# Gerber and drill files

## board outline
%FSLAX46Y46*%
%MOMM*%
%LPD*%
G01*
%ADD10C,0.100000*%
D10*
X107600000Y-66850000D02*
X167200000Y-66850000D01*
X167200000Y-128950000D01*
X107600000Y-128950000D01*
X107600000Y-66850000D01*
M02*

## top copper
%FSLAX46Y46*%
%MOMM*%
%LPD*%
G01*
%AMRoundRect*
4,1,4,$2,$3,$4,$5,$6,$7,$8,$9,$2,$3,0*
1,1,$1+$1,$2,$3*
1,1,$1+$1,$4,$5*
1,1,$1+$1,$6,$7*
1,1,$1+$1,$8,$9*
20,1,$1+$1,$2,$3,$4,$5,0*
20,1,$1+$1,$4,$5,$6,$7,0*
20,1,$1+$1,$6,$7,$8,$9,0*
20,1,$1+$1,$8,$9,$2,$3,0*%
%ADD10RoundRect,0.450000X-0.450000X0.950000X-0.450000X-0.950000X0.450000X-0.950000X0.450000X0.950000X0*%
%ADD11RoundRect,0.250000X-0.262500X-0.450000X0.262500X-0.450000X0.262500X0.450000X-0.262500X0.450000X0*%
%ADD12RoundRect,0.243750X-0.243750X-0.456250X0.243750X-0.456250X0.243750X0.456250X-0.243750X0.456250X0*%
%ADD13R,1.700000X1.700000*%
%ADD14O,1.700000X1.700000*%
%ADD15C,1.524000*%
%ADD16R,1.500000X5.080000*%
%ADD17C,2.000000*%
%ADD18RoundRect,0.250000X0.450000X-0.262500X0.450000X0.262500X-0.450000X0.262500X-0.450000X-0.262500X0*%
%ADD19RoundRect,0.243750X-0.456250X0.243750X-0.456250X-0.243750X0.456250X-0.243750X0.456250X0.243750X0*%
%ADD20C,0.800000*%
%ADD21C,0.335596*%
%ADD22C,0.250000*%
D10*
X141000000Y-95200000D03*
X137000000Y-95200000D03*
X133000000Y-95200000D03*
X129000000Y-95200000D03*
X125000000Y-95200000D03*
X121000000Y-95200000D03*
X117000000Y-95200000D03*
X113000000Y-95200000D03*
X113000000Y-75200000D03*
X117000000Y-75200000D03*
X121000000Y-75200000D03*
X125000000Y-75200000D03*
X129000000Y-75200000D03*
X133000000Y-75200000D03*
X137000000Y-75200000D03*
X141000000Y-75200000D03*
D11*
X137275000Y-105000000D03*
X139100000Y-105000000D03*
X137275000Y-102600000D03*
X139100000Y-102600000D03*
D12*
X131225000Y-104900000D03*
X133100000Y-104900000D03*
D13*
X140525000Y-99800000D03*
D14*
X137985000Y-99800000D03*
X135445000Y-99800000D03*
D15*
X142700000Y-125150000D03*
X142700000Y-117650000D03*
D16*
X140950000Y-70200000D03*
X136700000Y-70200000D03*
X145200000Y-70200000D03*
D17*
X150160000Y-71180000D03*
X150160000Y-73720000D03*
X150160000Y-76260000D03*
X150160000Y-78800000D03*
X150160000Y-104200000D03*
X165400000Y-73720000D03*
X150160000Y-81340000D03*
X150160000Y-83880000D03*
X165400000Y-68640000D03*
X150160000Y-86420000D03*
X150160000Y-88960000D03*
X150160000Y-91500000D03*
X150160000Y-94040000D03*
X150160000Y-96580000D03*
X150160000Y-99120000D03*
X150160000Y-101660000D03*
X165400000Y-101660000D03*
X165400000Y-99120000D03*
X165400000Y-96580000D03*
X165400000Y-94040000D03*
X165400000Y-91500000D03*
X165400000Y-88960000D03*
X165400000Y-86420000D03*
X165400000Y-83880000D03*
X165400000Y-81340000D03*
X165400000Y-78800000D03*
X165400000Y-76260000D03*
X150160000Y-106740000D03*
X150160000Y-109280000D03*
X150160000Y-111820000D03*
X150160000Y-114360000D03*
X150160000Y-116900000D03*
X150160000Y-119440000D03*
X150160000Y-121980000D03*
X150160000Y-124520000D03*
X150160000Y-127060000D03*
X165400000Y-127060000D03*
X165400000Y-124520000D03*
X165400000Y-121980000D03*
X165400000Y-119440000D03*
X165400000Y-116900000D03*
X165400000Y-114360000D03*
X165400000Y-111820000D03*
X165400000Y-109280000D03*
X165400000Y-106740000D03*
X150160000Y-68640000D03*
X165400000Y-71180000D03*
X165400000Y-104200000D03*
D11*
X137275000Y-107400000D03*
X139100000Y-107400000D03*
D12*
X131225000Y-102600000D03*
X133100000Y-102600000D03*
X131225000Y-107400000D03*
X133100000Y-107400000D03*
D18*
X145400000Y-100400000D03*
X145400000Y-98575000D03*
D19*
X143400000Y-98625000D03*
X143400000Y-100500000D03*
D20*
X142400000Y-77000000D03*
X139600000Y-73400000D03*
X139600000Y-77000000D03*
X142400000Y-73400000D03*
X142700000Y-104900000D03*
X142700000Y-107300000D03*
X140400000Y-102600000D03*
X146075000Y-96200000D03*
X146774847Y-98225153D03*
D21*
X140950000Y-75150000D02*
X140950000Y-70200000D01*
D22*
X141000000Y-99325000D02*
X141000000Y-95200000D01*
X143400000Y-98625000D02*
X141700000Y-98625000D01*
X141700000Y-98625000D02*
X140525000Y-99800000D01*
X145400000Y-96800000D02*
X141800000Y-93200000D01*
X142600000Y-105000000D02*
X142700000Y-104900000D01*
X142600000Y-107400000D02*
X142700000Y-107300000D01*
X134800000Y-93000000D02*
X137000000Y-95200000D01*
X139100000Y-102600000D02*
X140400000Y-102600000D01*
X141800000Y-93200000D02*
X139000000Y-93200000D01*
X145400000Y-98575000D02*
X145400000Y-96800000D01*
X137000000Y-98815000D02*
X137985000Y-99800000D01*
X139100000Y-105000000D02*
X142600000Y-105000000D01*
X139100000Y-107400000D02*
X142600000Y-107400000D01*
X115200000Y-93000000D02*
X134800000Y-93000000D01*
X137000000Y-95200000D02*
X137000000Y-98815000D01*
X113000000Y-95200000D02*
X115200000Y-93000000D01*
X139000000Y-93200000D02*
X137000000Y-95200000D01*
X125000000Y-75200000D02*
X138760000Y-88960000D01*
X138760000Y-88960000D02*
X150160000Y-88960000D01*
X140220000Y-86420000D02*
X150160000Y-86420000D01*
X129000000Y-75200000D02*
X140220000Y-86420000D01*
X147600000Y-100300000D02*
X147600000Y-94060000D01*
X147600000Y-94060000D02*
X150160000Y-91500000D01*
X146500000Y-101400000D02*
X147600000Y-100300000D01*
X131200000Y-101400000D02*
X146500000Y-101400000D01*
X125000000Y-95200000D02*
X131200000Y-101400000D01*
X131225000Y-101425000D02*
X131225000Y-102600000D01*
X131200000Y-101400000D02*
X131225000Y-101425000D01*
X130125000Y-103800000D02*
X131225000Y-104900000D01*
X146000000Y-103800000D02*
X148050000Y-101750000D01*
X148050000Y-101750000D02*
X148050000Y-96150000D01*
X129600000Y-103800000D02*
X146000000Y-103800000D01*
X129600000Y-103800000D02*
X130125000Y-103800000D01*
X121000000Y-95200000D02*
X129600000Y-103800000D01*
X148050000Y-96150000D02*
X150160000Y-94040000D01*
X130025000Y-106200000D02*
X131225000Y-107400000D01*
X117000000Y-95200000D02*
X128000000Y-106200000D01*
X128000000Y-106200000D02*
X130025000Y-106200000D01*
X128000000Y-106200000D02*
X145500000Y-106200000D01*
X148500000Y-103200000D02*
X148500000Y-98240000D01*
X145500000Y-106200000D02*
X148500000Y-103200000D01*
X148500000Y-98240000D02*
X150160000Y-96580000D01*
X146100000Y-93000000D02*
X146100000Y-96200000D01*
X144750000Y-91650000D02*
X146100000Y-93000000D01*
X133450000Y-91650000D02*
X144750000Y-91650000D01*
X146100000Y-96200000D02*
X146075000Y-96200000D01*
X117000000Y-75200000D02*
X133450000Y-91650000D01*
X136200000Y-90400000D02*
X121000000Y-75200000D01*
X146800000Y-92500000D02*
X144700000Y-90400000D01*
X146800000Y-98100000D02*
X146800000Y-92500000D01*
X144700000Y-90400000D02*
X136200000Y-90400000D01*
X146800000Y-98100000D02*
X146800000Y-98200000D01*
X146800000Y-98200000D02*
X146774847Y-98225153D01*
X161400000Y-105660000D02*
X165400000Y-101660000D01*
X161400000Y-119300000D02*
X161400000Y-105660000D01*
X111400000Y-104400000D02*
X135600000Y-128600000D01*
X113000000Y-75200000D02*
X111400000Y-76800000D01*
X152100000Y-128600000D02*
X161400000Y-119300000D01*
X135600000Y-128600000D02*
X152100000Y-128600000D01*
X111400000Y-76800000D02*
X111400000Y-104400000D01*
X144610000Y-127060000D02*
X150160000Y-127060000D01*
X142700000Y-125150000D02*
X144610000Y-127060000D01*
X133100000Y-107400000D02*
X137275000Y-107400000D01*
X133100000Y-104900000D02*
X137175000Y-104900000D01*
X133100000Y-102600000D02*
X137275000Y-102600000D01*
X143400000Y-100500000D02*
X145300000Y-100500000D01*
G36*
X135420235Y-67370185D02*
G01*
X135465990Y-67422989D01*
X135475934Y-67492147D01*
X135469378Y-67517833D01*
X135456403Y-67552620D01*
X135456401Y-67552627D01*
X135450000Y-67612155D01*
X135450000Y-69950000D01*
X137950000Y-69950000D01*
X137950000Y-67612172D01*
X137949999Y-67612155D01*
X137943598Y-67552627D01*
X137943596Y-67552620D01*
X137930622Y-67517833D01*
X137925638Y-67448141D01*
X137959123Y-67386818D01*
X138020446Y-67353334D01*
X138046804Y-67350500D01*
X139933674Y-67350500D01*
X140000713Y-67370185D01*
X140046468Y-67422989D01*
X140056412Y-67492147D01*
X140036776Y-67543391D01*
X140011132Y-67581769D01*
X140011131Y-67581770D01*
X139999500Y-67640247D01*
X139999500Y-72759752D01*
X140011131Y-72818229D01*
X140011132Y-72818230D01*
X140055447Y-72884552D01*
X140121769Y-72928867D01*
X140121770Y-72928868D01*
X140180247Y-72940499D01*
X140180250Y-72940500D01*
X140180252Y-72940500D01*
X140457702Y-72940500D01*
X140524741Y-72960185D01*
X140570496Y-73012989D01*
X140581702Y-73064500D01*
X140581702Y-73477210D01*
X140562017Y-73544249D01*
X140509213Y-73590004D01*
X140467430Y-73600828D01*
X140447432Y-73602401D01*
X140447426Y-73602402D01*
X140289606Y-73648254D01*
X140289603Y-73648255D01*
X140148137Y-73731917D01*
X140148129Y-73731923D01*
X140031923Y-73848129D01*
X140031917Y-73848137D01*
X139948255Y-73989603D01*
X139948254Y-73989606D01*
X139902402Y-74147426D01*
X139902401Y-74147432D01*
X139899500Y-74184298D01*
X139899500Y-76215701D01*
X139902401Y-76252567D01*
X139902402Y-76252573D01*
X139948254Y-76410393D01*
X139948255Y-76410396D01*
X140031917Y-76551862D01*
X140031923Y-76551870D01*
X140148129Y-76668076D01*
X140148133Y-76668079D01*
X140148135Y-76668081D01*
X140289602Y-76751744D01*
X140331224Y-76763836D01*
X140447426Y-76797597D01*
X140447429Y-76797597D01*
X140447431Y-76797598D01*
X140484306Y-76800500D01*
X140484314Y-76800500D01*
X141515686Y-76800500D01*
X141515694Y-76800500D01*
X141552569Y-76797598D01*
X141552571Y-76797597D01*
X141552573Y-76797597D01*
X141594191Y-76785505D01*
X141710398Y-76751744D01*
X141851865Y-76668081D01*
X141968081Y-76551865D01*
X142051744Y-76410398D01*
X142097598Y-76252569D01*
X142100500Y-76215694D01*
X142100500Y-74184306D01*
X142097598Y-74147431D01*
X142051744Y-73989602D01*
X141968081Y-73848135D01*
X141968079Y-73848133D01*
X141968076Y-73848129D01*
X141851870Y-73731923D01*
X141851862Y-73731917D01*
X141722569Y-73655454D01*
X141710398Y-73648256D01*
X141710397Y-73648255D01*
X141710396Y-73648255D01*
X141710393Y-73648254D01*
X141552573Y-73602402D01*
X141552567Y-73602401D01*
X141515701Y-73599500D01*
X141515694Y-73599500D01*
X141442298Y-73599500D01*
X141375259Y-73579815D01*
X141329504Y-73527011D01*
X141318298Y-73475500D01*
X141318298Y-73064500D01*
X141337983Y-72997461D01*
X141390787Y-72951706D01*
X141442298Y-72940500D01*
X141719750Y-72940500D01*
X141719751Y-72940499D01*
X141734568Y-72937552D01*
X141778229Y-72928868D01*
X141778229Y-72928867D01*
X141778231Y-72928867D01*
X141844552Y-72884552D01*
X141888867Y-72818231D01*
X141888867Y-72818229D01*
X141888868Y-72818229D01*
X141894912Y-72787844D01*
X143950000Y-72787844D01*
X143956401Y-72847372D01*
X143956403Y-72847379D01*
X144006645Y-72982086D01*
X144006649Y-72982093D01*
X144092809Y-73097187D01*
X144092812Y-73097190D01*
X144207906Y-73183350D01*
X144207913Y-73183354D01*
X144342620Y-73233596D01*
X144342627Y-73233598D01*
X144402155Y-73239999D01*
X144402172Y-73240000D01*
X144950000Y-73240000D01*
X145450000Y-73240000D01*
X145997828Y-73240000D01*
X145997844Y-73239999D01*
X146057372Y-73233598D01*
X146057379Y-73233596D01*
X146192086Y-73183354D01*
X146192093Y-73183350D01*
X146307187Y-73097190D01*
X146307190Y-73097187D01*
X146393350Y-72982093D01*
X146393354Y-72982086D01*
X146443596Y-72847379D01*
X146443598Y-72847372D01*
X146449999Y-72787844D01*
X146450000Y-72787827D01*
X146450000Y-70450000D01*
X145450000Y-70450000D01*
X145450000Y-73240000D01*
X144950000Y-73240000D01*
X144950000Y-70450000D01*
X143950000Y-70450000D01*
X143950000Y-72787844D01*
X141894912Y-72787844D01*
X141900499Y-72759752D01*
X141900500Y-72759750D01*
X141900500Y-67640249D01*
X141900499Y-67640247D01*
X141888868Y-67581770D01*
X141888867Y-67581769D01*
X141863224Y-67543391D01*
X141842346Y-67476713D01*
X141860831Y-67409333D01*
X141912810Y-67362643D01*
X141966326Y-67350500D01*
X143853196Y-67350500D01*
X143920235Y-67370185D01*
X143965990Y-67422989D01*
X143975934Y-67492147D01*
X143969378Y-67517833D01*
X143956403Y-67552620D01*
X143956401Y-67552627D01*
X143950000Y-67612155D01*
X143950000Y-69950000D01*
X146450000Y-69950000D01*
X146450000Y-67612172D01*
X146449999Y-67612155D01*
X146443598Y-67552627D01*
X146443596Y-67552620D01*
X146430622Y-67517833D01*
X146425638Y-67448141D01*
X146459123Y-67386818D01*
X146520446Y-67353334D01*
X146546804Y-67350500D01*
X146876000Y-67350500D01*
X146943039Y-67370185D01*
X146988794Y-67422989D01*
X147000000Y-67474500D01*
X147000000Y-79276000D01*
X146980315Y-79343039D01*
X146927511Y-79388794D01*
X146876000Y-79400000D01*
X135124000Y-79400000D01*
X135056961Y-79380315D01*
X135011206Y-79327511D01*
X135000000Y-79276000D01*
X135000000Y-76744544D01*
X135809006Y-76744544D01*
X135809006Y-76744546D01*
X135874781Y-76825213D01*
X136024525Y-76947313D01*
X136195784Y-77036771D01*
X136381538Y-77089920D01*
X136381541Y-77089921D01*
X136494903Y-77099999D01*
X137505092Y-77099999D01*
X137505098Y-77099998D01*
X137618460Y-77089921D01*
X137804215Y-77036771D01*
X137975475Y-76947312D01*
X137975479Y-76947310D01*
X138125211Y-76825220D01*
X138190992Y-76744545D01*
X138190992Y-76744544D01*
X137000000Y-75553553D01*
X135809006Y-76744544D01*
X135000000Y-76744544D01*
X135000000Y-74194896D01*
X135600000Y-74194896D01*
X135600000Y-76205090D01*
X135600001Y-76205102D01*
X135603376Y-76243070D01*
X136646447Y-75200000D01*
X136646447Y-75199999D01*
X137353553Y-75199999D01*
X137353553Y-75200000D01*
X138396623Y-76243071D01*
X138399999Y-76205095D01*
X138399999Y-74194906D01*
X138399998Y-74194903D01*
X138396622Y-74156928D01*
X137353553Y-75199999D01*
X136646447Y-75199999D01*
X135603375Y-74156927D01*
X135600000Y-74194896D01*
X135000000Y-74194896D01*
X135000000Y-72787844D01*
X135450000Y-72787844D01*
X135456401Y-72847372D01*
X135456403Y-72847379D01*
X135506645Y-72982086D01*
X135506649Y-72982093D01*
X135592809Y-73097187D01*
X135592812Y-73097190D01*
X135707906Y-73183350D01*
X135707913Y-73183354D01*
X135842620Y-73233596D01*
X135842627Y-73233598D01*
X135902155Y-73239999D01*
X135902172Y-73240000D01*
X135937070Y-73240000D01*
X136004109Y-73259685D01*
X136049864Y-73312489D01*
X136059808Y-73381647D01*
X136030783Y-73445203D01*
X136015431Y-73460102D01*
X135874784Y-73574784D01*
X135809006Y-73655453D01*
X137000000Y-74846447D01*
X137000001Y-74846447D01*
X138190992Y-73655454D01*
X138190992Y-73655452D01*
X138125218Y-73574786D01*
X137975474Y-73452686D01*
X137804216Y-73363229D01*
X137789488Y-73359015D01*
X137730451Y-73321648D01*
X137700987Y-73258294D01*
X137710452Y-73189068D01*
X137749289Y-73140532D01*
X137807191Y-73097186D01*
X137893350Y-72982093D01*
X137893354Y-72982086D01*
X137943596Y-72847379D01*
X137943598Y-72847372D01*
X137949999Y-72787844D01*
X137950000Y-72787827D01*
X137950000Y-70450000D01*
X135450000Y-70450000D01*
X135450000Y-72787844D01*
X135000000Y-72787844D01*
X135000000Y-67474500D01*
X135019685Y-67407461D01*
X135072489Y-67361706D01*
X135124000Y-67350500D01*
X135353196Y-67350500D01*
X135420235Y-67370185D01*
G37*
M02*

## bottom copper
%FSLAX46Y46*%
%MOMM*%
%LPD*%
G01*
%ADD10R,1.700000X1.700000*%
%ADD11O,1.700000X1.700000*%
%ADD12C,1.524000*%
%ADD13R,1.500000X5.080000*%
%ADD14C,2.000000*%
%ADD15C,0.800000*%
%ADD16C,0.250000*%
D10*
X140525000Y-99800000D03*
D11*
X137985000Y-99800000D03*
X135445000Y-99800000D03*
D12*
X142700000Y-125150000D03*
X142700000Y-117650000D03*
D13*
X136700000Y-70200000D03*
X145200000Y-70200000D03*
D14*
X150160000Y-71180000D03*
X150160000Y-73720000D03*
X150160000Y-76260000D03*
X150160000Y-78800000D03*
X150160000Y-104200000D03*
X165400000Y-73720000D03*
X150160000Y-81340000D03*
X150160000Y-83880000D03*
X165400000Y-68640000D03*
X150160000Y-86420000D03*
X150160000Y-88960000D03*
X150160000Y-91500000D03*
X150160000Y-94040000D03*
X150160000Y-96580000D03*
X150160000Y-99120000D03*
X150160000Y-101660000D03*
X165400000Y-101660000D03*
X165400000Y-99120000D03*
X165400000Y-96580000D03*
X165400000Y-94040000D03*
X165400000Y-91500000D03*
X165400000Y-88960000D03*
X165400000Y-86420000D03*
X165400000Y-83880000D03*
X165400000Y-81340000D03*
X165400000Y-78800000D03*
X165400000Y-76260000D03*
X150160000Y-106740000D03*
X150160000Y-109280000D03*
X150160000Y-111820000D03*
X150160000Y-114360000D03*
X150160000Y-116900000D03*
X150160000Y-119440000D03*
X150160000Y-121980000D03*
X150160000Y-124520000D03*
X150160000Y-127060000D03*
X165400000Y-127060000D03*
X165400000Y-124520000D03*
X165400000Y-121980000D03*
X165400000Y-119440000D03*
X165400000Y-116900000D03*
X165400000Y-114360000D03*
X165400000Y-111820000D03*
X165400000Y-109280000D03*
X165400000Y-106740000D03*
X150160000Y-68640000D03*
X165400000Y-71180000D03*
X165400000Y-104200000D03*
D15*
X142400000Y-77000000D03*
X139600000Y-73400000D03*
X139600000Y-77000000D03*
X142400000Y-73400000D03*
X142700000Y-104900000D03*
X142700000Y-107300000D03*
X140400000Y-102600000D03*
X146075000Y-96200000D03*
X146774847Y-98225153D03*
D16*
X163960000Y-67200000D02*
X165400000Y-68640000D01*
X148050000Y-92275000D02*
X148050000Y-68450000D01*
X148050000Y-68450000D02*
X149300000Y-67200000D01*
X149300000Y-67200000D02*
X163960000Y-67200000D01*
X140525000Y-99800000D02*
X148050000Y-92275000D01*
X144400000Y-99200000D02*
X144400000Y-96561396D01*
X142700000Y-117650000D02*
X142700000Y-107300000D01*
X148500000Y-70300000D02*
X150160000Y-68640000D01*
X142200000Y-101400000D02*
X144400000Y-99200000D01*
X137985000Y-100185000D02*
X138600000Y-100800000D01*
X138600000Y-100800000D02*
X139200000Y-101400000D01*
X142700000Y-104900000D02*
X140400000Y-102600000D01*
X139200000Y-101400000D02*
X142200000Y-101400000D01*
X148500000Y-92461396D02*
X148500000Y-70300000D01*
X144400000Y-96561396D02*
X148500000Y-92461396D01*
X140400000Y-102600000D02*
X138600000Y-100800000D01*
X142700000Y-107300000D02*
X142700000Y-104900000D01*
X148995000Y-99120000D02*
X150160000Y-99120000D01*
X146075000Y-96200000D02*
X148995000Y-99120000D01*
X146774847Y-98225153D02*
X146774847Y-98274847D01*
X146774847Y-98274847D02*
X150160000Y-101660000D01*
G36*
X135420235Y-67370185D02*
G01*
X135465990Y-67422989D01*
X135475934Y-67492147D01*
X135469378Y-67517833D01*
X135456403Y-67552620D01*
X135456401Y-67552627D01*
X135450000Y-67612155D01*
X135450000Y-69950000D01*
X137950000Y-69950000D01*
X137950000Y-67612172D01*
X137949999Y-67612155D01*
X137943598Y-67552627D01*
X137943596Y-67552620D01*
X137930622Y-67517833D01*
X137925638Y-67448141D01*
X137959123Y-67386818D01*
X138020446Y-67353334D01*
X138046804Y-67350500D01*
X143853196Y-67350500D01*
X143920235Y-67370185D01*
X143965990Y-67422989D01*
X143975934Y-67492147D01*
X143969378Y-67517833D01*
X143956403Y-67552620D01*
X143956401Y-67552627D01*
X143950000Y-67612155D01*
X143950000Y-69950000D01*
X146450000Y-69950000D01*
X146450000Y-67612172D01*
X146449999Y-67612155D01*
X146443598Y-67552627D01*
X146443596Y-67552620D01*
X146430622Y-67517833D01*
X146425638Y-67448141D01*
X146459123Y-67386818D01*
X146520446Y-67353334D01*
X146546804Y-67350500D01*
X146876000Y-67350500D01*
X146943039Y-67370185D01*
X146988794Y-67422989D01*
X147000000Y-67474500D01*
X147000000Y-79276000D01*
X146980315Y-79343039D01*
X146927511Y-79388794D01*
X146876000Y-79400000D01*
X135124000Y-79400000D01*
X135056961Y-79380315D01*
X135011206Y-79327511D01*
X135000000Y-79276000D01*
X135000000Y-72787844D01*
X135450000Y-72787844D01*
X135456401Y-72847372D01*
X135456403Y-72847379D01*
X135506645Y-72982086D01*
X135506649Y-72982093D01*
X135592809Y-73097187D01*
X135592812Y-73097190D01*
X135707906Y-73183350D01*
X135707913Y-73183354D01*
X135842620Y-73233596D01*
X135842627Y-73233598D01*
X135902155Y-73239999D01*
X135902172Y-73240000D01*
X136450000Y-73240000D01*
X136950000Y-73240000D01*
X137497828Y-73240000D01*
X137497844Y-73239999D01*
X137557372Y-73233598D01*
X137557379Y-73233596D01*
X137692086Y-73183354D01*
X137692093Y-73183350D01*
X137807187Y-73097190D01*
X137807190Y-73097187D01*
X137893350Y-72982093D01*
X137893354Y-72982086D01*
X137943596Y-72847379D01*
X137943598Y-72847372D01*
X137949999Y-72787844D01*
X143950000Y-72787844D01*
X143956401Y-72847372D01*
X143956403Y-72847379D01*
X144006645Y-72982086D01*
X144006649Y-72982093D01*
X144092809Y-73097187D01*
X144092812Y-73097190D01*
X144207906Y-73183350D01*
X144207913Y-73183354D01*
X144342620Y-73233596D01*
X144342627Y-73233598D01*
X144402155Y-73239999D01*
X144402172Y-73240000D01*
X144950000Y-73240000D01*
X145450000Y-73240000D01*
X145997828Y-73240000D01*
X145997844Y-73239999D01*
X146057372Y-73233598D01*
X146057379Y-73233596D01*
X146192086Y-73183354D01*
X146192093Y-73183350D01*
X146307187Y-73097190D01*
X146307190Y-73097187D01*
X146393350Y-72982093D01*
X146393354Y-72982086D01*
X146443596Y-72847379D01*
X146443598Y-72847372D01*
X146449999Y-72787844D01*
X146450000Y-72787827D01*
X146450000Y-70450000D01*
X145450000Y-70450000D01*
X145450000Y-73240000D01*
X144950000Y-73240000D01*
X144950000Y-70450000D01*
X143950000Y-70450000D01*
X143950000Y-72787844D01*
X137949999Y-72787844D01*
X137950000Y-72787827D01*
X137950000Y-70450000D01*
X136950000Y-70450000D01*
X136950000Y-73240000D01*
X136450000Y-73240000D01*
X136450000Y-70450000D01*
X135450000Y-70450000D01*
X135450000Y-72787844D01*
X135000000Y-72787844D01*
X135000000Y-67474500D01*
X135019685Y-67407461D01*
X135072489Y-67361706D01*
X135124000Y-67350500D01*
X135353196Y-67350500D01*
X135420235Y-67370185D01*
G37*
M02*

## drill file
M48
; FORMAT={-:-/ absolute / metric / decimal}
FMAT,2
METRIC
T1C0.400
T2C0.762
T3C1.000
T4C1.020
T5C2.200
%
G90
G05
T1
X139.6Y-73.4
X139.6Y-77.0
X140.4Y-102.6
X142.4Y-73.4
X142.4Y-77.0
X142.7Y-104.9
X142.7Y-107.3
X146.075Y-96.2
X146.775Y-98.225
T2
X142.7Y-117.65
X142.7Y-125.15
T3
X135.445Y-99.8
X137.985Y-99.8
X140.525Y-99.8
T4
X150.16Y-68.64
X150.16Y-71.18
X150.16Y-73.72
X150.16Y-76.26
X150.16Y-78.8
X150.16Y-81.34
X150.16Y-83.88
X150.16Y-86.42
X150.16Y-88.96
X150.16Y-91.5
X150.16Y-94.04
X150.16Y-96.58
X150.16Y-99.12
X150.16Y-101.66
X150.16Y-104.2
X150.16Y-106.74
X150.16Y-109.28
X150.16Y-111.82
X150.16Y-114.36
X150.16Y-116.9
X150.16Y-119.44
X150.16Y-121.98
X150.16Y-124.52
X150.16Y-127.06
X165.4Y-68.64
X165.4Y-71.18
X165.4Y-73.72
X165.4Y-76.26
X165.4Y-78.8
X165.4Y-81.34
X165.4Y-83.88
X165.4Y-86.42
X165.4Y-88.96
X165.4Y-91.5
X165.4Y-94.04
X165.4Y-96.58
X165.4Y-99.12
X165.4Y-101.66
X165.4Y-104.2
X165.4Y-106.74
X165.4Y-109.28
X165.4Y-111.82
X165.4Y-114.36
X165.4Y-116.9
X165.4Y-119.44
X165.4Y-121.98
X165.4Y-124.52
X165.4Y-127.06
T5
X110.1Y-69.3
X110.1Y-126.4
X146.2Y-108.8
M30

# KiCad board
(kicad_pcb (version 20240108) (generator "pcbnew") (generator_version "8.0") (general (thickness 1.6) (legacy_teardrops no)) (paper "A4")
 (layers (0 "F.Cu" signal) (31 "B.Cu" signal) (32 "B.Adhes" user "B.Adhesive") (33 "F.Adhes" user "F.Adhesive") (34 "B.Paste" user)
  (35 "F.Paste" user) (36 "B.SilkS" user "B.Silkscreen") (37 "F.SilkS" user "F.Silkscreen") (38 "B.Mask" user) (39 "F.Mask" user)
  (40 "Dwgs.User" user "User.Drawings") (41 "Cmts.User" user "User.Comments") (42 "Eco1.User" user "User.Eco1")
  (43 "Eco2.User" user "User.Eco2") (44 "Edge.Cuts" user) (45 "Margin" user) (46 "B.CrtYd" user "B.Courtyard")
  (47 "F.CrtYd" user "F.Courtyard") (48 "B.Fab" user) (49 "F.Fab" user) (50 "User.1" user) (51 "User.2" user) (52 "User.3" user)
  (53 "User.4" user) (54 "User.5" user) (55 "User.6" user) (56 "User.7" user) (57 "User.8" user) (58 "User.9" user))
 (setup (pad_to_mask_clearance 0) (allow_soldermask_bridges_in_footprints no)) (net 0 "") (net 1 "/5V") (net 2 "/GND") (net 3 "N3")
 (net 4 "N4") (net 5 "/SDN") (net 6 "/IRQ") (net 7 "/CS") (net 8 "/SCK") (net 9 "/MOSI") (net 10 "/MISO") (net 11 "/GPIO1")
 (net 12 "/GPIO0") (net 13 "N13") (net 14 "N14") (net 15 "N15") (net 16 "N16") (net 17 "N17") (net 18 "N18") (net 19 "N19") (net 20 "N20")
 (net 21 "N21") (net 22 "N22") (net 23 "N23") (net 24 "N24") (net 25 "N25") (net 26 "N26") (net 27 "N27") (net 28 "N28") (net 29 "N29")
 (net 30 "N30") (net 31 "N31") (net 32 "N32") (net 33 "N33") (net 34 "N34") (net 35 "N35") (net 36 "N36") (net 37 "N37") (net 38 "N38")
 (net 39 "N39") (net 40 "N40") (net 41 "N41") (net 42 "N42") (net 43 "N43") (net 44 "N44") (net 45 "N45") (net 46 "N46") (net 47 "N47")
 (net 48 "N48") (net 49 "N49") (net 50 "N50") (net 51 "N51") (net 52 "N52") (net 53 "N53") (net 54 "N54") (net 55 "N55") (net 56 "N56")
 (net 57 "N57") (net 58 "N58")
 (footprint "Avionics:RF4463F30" (layer "F.Cu") (at 127 85.2 180)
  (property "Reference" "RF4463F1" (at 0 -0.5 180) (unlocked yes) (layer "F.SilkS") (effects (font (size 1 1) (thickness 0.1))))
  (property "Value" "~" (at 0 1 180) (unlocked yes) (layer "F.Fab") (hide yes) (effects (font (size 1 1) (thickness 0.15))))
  (pad "1" smd roundrect (at -14 -10 270) (size 2.8 1.8) (layers "F.Cu" "F.Paste" "F.Mask") (roundrect_rratio 0.25) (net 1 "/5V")
   (thermal_bridge_angle 45))
  (pad "2" smd roundrect (at -10 -10 270) (size 2.8 1.8) (layers "F.Cu" "F.Paste" "F.Mask") (roundrect_rratio 0.25) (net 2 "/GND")
   (thermal_bridge_angle 45))
  (pad "3" smd roundrect (at -6 -10 270) (size 2.8 1.8) (layers "F.Cu" "F.Paste" "F.Mask") (roundrect_rratio 0.25) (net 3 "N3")
   (thermal_bridge_angle 45))
  (pad "4" smd roundrect (at -2 -10 270) (size 2.8 1.8) (layers "F.Cu" "F.Paste" "F.Mask") (roundrect_rratio 0.25) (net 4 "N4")
   (thermal_bridge_angle 45))
  (pad "5" smd roundrect (at 2 -10 270) (size 2.8 1.8) (layers "F.Cu" "F.Paste" "F.Mask") (roundrect_rratio 0.25) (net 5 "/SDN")
   (thermal_bridge_angle 45))
  (pad "6" smd roundrect (at 6 -10 270) (size 2.8 1.8) (layers "F.Cu" "F.Paste" "F.Mask") (roundrect_rratio 0.25) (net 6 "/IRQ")
   (thermal_bridge_angle 45))
  (pad "7" smd roundrect (at 10 -10 270) (size 2.8 1.8) (layers "F.Cu" "F.Paste" "F.Mask") (roundrect_rratio 0.25) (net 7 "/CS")
   (thermal_bridge_angle 45))
  (pad "8" smd roundrect (at 14 -10 270) (size 2.8 1.8) (layers "F.Cu" "F.Paste" "F.Mask") (roundrect_rratio 0.25) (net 2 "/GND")
   (thermal_bridge_angle 45))
  (pad "9" smd roundrect (at 14 10 270) (size 2.8 1.8) (layers "F.Cu" "F.Paste" "F.Mask") (roundrect_rratio 0.25) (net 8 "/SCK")
   (thermal_bridge_angle 45))
  (pad "10" smd roundrect (at 10 10 270) (size 2.8 1.8) (layers "F.Cu" "F.Paste" "F.Mask") (roundrect_rratio 0.25) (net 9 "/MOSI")
   (thermal_bridge_angle 45))
  (pad "11" smd roundrect (at 6 10 270) (size 2.8 1.8) (layers "F.Cu" "F.Paste" "F.Mask") (roundrect_rratio 0.25) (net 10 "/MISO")
   (thermal_bridge_angle 45))
  (pad "12" smd roundrect (at 2 10 270) (size 2.8 1.8) (layers "F.Cu" "F.Paste" "F.Mask") (roundrect_rratio 0.25) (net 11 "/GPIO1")
   (thermal_bridge_angle 45))
  (pad "13" smd roundrect (at -2 10 270) (size 2.8 1.8) (layers "F.Cu" "F.Paste" "F.Mask") (roundrect_rratio 0.25) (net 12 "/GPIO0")
   (thermal_bridge_angle 45))
  (pad "14" smd roundrect (at -6 10 270) (size 2.8 1.8) (layers "F.Cu" "F.Paste" "F.Mask") (roundrect_rratio 0.25) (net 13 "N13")
   (thermal_bridge_angle 45))
  (pad "15" smd roundrect (at -10 10 270) (size 2.8 1.8) (layers "F.Cu" "F.Paste" "F.Mask") (roundrect_rratio 0.25) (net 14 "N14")
   (thermal_bridge_angle 45))
  (pad "16" smd roundrect (at -14 10 270) (size 2.8 1.8) (layers "F.Cu" "F.Paste" "F.Mask") (roundrect_rratio 0.25) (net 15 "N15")
   (thermal_bridge_angle 45)))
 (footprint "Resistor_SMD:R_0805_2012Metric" (layer "F.Cu") (at 138.1875 105)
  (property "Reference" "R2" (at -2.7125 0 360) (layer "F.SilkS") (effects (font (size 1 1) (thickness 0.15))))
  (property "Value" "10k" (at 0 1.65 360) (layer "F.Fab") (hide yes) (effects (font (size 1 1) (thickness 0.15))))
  (pad "1" smd roundrect (at -0.9125 0) (size 1.025 1.4) (layers "F.Cu" "F.Paste" "F.Mask") (roundrect_rratio 0.243902) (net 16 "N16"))
  (pad "2" smd roundrect (at 0.9125 0) (size 1.025 1.4) (layers "F.Cu" "F.Paste" "F.Mask") (roundrect_rratio 0.243902) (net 2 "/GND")))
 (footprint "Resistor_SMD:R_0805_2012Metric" (layer "F.Cu") (at 138.1875 102.6)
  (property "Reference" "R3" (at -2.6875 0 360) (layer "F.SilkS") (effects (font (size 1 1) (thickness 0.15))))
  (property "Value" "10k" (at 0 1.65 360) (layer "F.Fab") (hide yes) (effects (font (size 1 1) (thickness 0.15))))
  (pad "1" smd roundrect (at -0.9125 0) (size 1.025 1.4) (layers "F.Cu" "F.Paste" "F.Mask") (roundrect_rratio 0.243902) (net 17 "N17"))
  (pad "2" smd roundrect (at 0.9125 0) (size 1.025 1.4) (layers "F.Cu" "F.Paste" "F.Mask") (roundrect_rratio 0.243902) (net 2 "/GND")))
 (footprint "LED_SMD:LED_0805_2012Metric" (layer "F.Cu") (at 132.1625 104.9)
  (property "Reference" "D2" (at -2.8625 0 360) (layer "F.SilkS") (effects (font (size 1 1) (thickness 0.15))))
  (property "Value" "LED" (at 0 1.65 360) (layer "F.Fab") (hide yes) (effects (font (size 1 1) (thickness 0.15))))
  (pad "1" smd roundrect (at -0.9375 0) (size 0.975 1.4) (layers "F.Cu" "F.Paste" "F.Mask") (roundrect_rratio 0.25) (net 6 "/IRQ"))
  (pad "2" smd roundrect (at 0.9375 0) (size 0.975 1.4) (layers "F.Cu" "F.Paste" "F.Mask") (roundrect_rratio 0.25) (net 16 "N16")))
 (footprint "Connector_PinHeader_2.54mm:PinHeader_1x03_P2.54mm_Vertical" (layer "F.Cu") (at 140.525 99.8 -90)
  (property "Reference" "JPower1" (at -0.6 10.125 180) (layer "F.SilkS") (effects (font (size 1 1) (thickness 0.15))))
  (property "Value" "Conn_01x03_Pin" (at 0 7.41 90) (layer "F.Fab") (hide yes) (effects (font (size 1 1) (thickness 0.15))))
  (pad "1" thru_hole rect (at 0 0 270) (size 1.7 1.7) (drill 1) (layers "*.Cu" "*.Mask") (remove_unused_layers no) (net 1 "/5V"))
  (pad "2" thru_hole oval (at 0 2.54 270) (size 1.7 1.7) (drill 1) (layers "*.Cu" "*.Mask") (remove_unused_layers no) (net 2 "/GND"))
  (pad "3" thru_hole oval (at 0 5.08 270) (size 1.7 1.7) (drill 1) (layers "*.Cu" "*.Mask") (remove_unused_layers no) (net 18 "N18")))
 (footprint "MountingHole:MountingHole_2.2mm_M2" (layer "F.Cu") (at 110.1 69.3)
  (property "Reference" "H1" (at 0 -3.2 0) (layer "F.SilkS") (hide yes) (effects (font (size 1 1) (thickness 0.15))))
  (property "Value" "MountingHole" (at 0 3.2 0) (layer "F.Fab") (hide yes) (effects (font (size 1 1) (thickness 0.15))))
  (pad "" np_thru_hole circle (at 0 0) (size 2.2 2.2) (drill 2.2) (layers "*.Cu" "*.Mask")))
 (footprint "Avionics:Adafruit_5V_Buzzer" (layer "F.Cu") (at 147.2 121.4 90)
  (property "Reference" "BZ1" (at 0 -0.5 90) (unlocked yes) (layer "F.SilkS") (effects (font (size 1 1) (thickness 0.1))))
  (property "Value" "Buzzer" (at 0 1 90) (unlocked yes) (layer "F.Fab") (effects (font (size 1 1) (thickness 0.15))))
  (pad "1" thru_hole circle (at -3.75 -4.5 90) (size 1.524 1.524) (drill 0.762) (layers "*.Cu" "*.Mask") (remove_unused_layers no)
   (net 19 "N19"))
  (pad "2" thru_hole circle (at 3.75 -4.5 90) (size 1.524 1.524) (drill 0.762) (layers "*.Cu" "*.Mask") (remove_unused_layers no)
   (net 2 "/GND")))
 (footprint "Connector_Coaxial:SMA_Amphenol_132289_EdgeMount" (layer "F.Cu") (at 140.95 70.2 90)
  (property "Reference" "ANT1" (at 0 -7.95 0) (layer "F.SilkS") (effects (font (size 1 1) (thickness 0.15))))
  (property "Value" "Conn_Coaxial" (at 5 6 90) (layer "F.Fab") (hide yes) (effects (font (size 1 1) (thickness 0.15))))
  (pad "1" smd rect (at 0 0 180) (size 1.5 5.08) (layers "F.Cu" "F.Paste" "F.Mask") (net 15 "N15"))
  (pad "2" smd rect (at 0 -4.25 180) (size 1.5 5.08) (layers "F.Cu" "F.Paste" "F.Mask") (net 14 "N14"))
  (pad "2" smd rect (at 0 -4.25 180) (size 1.5 5.08) (layers "B.Cu" "B.Paste" "B.Mask") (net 14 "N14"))
  (pad "2" smd rect (at 0 4.25 180) (size 1.5 5.08) (layers "F.Cu" "F.Paste" "F.Mask") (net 14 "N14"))
  (pad "2" smd rect (at 0 4.25 180) (size 1.5 5.08) (layers "B.Cu" "B.Paste" "B.Mask") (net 14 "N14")))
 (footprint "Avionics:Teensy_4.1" (layer "F.Cu") (at 157.78 97.85)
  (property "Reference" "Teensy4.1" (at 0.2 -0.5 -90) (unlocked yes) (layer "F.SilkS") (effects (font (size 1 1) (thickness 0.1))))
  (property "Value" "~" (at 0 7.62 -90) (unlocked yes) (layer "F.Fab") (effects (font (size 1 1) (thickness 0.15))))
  (pad "0" thru_hole circle (at -7.62 -26.67) (size 2 2) (drill 1.02) (layers "*.Cu" "*.Mask") (remove_unused_layers no) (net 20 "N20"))
  (pad "1" thru_hole circle (at -7.62 -24.13) (size 2 2) (drill 1.02) (layers "*.Cu" "*.Mask") (remove_unused_layers no) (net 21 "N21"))
  (pad "2" thru_hole circle (at -7.62 -21.59) (size 2 2) (drill 1.02) (layers "*.Cu" "*.Mask") (remove_unused_layers no) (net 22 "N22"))
  (pad "3" thru_hole circle (at -7.62 -19.05) (size 2 2) (drill 1.02) (layers "*.Cu" "*.Mask") (remove_unused_layers no) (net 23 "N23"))
  (pad "3V" thru_hole circle (at -7.62 6.35) (size 2 2) (drill 1.02) (layers "*.Cu" "*.Mask") (remove_unused_layers no) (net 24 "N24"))
  (pad "3V1" thru_hole circle (at 7.62 -24.13) (size 2 2) (drill 1.02) (layers "*.Cu" "*.Mask") (remove_unused_layers no) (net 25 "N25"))
  (pad "4" thru_hole circle (at -7.62 -16.51) (size 2 2) (drill 1.02) (layers "*.Cu" "*.Mask") (remove_unused_layers no) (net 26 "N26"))
  (pad "5" thru_hole circle (at -7.62 -13.97) (size 2 2) (drill 1.02) (layers "*.Cu" "*.Mask") (remove_unused_layers no) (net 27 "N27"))
  (pad "5V" thru_hole circle (at 7.62 -29.21) (size 2 2) (drill 1.02) (layers "*.Cu" "*.Mask") (remove_unused_layers no) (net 1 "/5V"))
  (pad "6" thru_hole circle (at -7.62 -11.43) (size 2 2) (drill 1.02) (layers "*.Cu" "*.Mask") (remove_unused_layers no) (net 12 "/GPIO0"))
  (pad "7" thru_hole circle (at -7.62 -8.89) (size 2 2) (drill 1.02) (layers "*.Cu" "*.Mask") (remove_unused_layers no) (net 11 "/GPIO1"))
  (pad "8" thru_hole circle (at -7.62 -6.35) (size 2 2) (drill 1.02) (layers "*.Cu" "*.Mask") (remove_unused_layers no) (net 5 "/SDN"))
  (pad "9" thru_hole circle (at -7.62 -3.81) (size 2 2) (drill 1.02) (layers "*.Cu" "*.Mask") (remove_unused_layers no) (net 6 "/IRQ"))
  (pad "10" thru_hole circle (at -7.62 -1.27) (size 2 2) (drill 1.02) (layers "*.Cu" "*.Mask") (remove_unused_layers no) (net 7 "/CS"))
  (pad "11" thru_hole circle (at -7.62 1.27) (size 2 2) (drill 1.02) (layers "*.Cu" "*.Mask") (remove_unused_layers no) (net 9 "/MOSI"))
  (pad "12" thru_hole circle (at -7.62 3.81) (size 2 2) (drill 1.02) (layers "*.Cu" "*.Mask") (remove_unused_layers no) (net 10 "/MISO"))
  (pad "13" thru_hole circle (at 7.62 3.81) (size 2 2) (drill 1.02) (layers "*.Cu" "*.Mask") (remove_unused_layers no) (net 8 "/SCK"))
  (pad "14" thru_hole circle (at 7.62 1.27) (size 2 2) (drill 1.02) (layers "*.Cu" "*.Mask") (remove_unused_layers no) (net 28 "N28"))
  (pad "15" thru_hole circle (at 7.62 -1.27) (size 2 2) (drill 1.02) (layers "*.Cu" "*.Mask") (remove_unused_layers no) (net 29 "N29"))
  (pad "16" thru_hole circle (at 7.62 -3.81) (size 2 2) (drill 1.02) (layers "*.Cu" "*.Mask") (remove_unused_layers no) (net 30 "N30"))
  (pad "17" thru_hole circle (at 7.62 -6.35) (size 2 2) (drill 1.02) (layers "*.Cu" "*.Mask") (remove_unused_layers no) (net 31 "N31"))
  (pad "18" thru_hole circle (at 7.62 -8.89) (size 2 2) (drill 1.02) (layers "*.Cu" "*.Mask") (remove_unused_layers no) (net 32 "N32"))
  (pad "19" thru_hole circle (at 7.62 -11.43) (size 2 2) (drill 1.02) (layers "*.Cu" "*.Mask") (remove_unused_layers no) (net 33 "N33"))
  (pad "20" thru_hole circle (at 7.62 -13.97) (size 2 2) (drill 1.02) (layers "*.Cu" "*.Mask") (remove_unused_layers no) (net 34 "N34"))
  (pad "21" thru_hole circle (at 7.62 -16.51) (size 2 2) (drill 1.02) (layers "*.Cu" "*.Mask") (remove_unused_layers no) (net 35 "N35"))
  (pad "22" thru_hole circle (at 7.62 -19.05) (size 2 2) (drill 1.02) (layers "*.Cu" "*.Mask") (remove_unused_layers no) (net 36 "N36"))
  (pad "23" thru_hole circle (at 7.62 -21.59) (size 2 2) (drill 1.02) (layers "*.Cu" "*.Mask") (remove_unused_layers no) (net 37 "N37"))
  (pad "24" thru_hole circle (at -7.62 8.89) (size 2 2) (drill 1.02) (layers "*.Cu" "*.Mask") (remove_unused_layers no) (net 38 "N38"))
  (pad "25" thru_hole circle (at -7.62 11.43) (size 2 2) (drill 1.02) (layers "*.Cu" "*.Mask") (remove_unused_layers no) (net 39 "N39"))
  (pad "26" thru_hole circle (at -7.62 13.97) (size 2 2) (drill 1.02) (layers "*.Cu" "*.Mask") (remove_unused_layers no) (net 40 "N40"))
  (pad "27" thru_hole circle (at -7.62 16.51) (size 2 2) (drill 1.02) (layers "*.Cu" "*.Mask") (remove_unused_layers no) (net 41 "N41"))
  (pad "28" thru_hole circle (at -7.62 19.05) (size 2 2) (drill 1.02) (layers "*.Cu" "*.Mask") (remove_unused_layers no) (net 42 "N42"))
  (pad "29" thru_hole circle (at -7.62 21.59) (size 2 2) (drill 1.02) (layers "*.Cu" "*.Mask") (remove_unused_layers no) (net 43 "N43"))
  (pad "30" thru_hole circle (at -7.62 24.13) (size 2 2) (drill 1.02) (layers "*.Cu" "*.Mask") (remove_unused_layers no) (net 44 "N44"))
  (pad "31" thru_hole circle (at -7.62 26.67) (size 2 2) (drill 1.02) (layers "*.Cu" "*.Mask") (remove_unused_layers no) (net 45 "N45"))
  (pad "32" thru_hole circle (at -7.62 29.21) (size 2 2) (drill 1.02) (layers "*.Cu" "*.Mask") (remove_unused_layers no) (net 19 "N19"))
  (pad "33" thru_hole circle (at 7.62 29.21) (size 2 2) (drill 1.02) (layers "*.Cu" "*.Mask") (remove_unused_layers no) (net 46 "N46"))
  (pad "34" thru_hole circle (at 7.62 26.67) (size 2 2) (drill 1.02) (layers "*.Cu" "*.Mask") (remove_unused_layers no) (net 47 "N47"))
  (pad "35" thru_hole circle (at 7.62 24.13) (size 2 2) (drill 1.02) (layers "*.Cu" "*.Mask") (remove_unused_layers no) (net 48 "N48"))
  (pad "36" thru_hole circle (at 7.62 21.59) (size 2 2) (drill 1.02) (layers "*.Cu" "*.Mask") (remove_unused_layers no) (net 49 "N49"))
  (pad "37" thru_hole circle (at 7.62 19.05) (size 2 2) (drill 1.02) (layers "*.Cu" "*.Mask") (remove_unused_layers no) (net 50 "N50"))
  (pad "38" thru_hole circle (at 7.62 16.51) (size 2 2) (drill 1.02) (layers "*.Cu" "*.Mask") (remove_unused_layers no) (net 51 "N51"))
  (pad "39" thru_hole circle (at 7.62 13.97) (size 2 2) (drill 1.02) (layers "*.Cu" "*.Mask") (remove_unused_layers no) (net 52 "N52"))
  (pad "40" thru_hole circle (at 7.62 11.43) (size 2 2) (drill 1.02) (layers "*.Cu" "*.Mask") (remove_unused_layers no) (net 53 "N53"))
  (pad "41" thru_hole circle (at 7.62 8.89) (size 2 2) (drill 1.02) (layers "*.Cu" "*.Mask") (remove_unused_layers no) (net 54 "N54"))
  (pad "G" thru_hole circle (at -7.62 -29.21) (size 2 2) (drill 1.02) (layers "*.Cu" "*.Mask") (remove_unused_layers no) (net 2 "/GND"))
  (pad "G1" thru_hole circle (at 7.62 -26.67) (size 2 2) (drill 1.02) (layers "*.Cu" "*.Mask") (remove_unused_layers no) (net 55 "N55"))
  (pad "G2" thru_hole circle (at 7.62 6.35) (size 2 2) (drill 1.02) (layers "*.Cu" "*.Mask") (remove_unused_layers no) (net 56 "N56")))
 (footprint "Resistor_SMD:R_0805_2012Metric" (layer "F.Cu") (at 138.1875 107.4)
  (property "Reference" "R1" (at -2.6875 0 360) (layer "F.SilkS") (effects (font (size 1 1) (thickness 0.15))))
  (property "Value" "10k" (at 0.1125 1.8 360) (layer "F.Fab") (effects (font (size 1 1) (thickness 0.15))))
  (pad "1" smd roundrect (at -0.9125 0) (size 1.025 1.4) (layers "F.Cu" "F.Paste" "F.Mask") (roundrect_rratio 0.243902) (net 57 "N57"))
  (pad "2" smd roundrect (at 0.9125 0) (size 1.025 1.4) (layers "F.Cu" "F.Paste" "F.Mask") (roundrect_rratio 0.243902) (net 2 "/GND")))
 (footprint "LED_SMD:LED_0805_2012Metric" (layer "F.Cu") (at 132.1625 102.6)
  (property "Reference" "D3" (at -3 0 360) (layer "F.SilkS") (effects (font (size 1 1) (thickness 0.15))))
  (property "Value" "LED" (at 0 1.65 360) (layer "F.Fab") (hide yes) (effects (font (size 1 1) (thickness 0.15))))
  (pad "1" smd roundrect (at -0.9375 0) (size 0.975 1.4) (layers "F.Cu" "F.Paste" "F.Mask") (roundrect_rratio 0.25) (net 5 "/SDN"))
  (pad "2" smd roundrect (at 0.9375 0) (size 0.975 1.4) (layers "F.Cu" "F.Paste" "F.Mask") (roundrect_rratio 0.25) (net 17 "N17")))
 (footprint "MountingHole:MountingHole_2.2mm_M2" (layer "F.Cu") (at 110.1 126.4)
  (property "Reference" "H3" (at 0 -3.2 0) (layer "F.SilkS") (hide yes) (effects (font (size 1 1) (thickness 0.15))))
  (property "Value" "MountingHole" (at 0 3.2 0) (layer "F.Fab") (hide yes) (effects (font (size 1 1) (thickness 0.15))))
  (pad "" np_thru_hole circle (at 0 0) (size 2.2 2.2) (drill 2.2) (layers "*.Cu" "*.Mask")))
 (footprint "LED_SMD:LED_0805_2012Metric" (layer "F.Cu") (at 132.1625 107.4)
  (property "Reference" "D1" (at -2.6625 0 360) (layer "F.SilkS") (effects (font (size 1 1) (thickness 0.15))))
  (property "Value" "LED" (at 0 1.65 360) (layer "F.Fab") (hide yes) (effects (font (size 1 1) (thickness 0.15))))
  (pad "1" smd roundrect (at -0.9375 0) (size 0.975 1.4) (layers "F.Cu" "F.Paste" "F.Mask") (roundrect_rratio 0.25) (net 7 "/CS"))
  (pad "2" smd roundrect (at 0.9375 0) (size 0.975 1.4) (layers "F.Cu" "F.Paste" "F.Mask") (roundrect_rratio 0.25) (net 57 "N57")))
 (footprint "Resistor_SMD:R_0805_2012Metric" (layer "F.Cu") (at 145.4 99.4875 90)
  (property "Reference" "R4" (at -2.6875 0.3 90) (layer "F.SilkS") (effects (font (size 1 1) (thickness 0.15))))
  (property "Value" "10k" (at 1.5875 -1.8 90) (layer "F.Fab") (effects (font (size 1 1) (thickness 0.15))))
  (pad "1" smd roundrect (at -0.9125 0 90) (size 1.025 1.4) (layers "F.Cu" "F.Paste" "F.Mask") (roundrect_rratio 0.243902) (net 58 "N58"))
  (pad "2" smd roundrect (at 0.9125 0 90) (size 1.025 1.4) (layers "F.Cu" "F.Paste" "F.Mask") (roundrect_rratio 0.243902) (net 2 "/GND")))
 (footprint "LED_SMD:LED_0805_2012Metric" (layer "F.Cu") (at 143.4 99.5625 -90)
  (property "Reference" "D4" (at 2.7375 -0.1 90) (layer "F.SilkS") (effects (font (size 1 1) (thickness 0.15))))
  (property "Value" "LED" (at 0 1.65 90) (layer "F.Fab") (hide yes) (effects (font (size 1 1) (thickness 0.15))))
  (pad "1" smd roundrect (at -0.9375 0 270) (size 0.975 1.4) (layers "F.Cu" "F.Paste" "F.Mask") (roundrect_rratio 0.25) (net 1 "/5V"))
  (pad "2" smd roundrect (at 0.9375 0 270) (size 0.975 1.4) (layers "F.Cu" "F.Paste" "F.Mask") (roundrect_rratio 0.25) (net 58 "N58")))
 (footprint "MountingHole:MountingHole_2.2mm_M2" (layer "F.Cu") (at 146.2 108.8)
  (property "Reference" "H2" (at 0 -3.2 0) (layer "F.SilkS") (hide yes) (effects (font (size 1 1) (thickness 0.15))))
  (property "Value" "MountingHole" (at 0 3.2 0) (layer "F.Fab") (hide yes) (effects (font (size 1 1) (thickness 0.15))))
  (pad "" np_thru_hole circle (at 0 0) (size 2.2 2.2) (drill 2.2) (layers "*.Cu" "*.Mask")))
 (gr_rect (start 107.6 66.85) (end 167.2 128.95) (stroke (width 0.1) (type default)) (fill none) (layer "Edge.Cuts"))
 (segment (start 140.95 75.15) (end 140.95 70.2) (width 0.335596) (layer "F.Cu") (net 15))
 (via (at 142.4 77) (size 0.8) (drill 0.4) (layers "F.Cu" "B.Cu") (free yes) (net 14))
 (via (at 139.6 73.4) (size 0.8) (drill 0.4) (layers "F.Cu" "B.Cu") (free yes) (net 14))
 (via (at 139.6 77) (size 0.8) (drill 0.4) (layers "F.Cu" "B.Cu") (free yes) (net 14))
 (via (at 142.4 73.4) (size 0.8) (drill 0.4) (layers "F.Cu" "B.Cu") (free yes) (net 14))
 (segment (start 141 99.325) (end 141 95.2) (width 0.25) (layer "F.Cu") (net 1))
 (segment (start 143.4 98.625) (end 141.7 98.625) (width 0.25) (layer "F.Cu") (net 1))
 (segment (start 141.7 98.625) (end 140.525 99.8) (width 0.25) (layer "F.Cu") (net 1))
 (segment (start 163.96 67.2) (end 165.4 68.64) (width 0.25) (layer "B.Cu") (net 1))
 (segment (start 148.05 92.275) (end 148.05 68.45) (width 0.25) (layer "B.Cu") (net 1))
 (segment (start 148.05 68.45) (end 149.3 67.2) (width 0.25) (layer "B.Cu") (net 1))
 (segment (start 149.3 67.2) (end 163.96 67.2) (width 0.25) (layer "B.Cu") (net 1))
 (segment (start 140.525 99.8) (end 148.05 92.275) (width 0.25) (layer "B.Cu") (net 1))
 (segment (start 145.4 96.8) (end 141.8 93.2) (width 0.25) (layer "F.Cu") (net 2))
 (segment (start 142.6 105) (end 142.7 104.9) (width 0.25) (layer "F.Cu") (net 2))
 (segment (start 142.6 107.4) (end 142.7 107.3) (width 0.25) (layer "F.Cu") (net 2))
 (segment (start 134.8 93) (end 137 95.2) (width 0.25) (layer "F.Cu") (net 2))
 (segment (start 139.1 102.6) (end 140.4 102.6) (width 0.25) (layer "F.Cu") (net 2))
 (segment (start 141.8 93.2) (end 139 93.2) (width 0.25) (layer "F.Cu") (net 2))
 (segment (start 145.4 98.575) (end 145.4 96.8) (width 0.25) (layer "F.Cu") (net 2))
 (segment (start 137 98.815) (end 137.985 99.8) (width 0.25) (layer "F.Cu") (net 2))
 (segment (start 139.1 105) (end 142.6 105) (width 0.25) (layer "F.Cu") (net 2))
 (segment (start 139.1 107.4) (end 142.6 107.4) (width 0.25) (layer "F.Cu") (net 2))
 (segment (start 115.2 93) (end 134.8 93) (width 0.25) (layer "F.Cu") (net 2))
 (segment (start 137 95.2) (end 137 98.815) (width 0.25) (layer "F.Cu") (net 2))
 (segment (start 113 95.2) (end 115.2 93) (width 0.25) (layer "F.Cu") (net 2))
 (segment (start 139 93.2) (end 137 95.2) (width 0.25) (layer "F.Cu") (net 2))
 (via (at 142.7 104.9) (size 0.8) (drill 0.4) (layers "F.Cu" "B.Cu") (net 2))
 (via (at 142.7 107.3) (size 0.8) (drill 0.4) (layers "F.Cu" "B.Cu") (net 2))
 (via (at 140.4 102.6) (size 0.8) (drill 0.4) (layers "F.Cu" "B.Cu") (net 2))
 (segment (start 144.4 99.2) (end 144.4 96.561396) (width 0.25) (layer "B.Cu") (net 2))
 (segment (start 142.7 117.65) (end 142.7 107.3) (width 0.25) (layer "B.Cu") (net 2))
 (segment (start 148.5 70.3) (end 150.16 68.64) (width 0.25) (layer "B.Cu") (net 2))
 (segment (start 142.2 101.4) (end 144.4 99.2) (width 0.25) (layer "B.Cu") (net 2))
 (segment (start 137.985 100.185) (end 138.6 100.8) (width 0.25) (layer "B.Cu") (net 2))
 (segment (start 138.6 100.8) (end 139.2 101.4) (width 0.25) (layer "B.Cu") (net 2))
 (segment (start 142.7 104.9) (end 140.4 102.6) (width 0.25) (layer "B.Cu") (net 2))
 (segment (start 139.2 101.4) (end 142.2 101.4) (width 0.25) (layer "B.Cu") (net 2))
 (segment (start 148.5 92.461396) (end 148.5 70.3) (width 0.25) (layer "B.Cu") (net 2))
 (segment (start 144.4 96.561396) (end 148.5 92.461396) (width 0.25) (layer "B.Cu") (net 2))
 (segment (start 140.4 102.6) (end 138.6 100.8) (width 0.25) (layer "B.Cu") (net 2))
 (segment (start 142.7 107.3) (end 142.7 104.9) (width 0.25) (layer "B.Cu") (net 2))
 (segment (start 125 75.2) (end 138.76 88.96) (width 0.25) (layer "F.Cu") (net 11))
 (segment (start 138.76 88.96) (end 150.16 88.96) (width 0.25) (layer "F.Cu") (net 11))
 (segment (start 140.22 86.42) (end 150.16 86.42) (width 0.25) (layer "F.Cu") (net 12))
 (segment (start 129 75.2) (end 140.22 86.42) (width 0.25) (layer "F.Cu") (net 12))
 (segment (start 147.6 100.3) (end 147.6 94.06) (width 0.25) (layer "F.Cu") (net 5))
 (segment (start 147.6 94.06) (end 150.16 91.5) (width 0.25) (layer "F.Cu") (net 5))
 (segment (start 146.5 101.4) (end 147.6 100.3) (width 0.25) (layer "F.Cu") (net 5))
 (segment (start 131.2 101.4) (end 146.5 101.4) (width 0.25) (layer "F.Cu") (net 5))
 (segment (start 125 95.2) (end 131.2 101.4) (width 0.25) (layer "F.Cu") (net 5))
 (segment (start 131.225 101.425) (end 131.225 102.6) (width 0.25) (layer "F.Cu") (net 5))
 (segment (start 131.2 101.4) (end 131.225 101.425) (width 0.25) (layer "F.Cu") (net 5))
 (segment (start 130.125 103.8) (end 131.225 104.9) (width 0.25) (layer "F.Cu") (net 6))
 (segment (start 146 103.8) (end 148.05 101.75) (width 0.25) (layer "F.Cu") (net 6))
 (segment (start 148.05 101.75) (end 148.05 96.15) (width 0.25) (layer "F.Cu") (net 6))
 (segment (start 129.6 103.8) (end 146 103.8) (width 0.25) (layer "F.Cu") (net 6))
 (segment (start 129.6 103.8) (end 130.125 103.8) (width 0.25) (layer "F.Cu") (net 6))
 (segment (start 121 95.2) (end 129.6 103.8) (width 0.25) (layer "F.Cu") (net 6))
 (segment (start 148.05 96.15) (end 150.16 94.04) (width 0.25) (layer "F.Cu") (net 6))
 (segment (start 130.025 106.2) (end 131.225 107.4) (width 0.25) (layer "F.Cu") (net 7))
 (segment (start 117 95.2) (end 128 106.2) (width 0.25) (layer "F.Cu") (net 7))
 (segment (start 128 106.2) (end 130.025 106.2) (width 0.25) (layer "F.Cu") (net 7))
 (segment (start 128 106.2) (end 145.5 106.2) (width 0.25) (layer "F.Cu") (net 7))
 (segment (start 148.5 103.2) (end 148.5 98.24) (width 0.25) (layer "F.Cu") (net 7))
 (segment (start 145.5 106.2) (end 148.5 103.2) (width 0.25) (layer "F.Cu") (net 7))
 (segment (start 148.5 98.24) (end 150.16 96.58) (width 0.25) (layer "F.Cu") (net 7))
 (segment (start 146.1 93) (end 146.1 96.2) (width 0.25) (layer "F.Cu") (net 9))
 (segment (start 144.75 91.65) (end 146.1 93) (width 0.25) (layer "F.Cu") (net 9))
 (segment (start 133.45 91.65) (end 144.75 91.65) (width 0.25) (layer "F.Cu") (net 9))
 (segment (start 146.1 96.2) (end 146.075 96.2) (width 0.25) (layer "F.Cu") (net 9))
 (segment (start 117 75.2) (end 133.45 91.65) (width 0.25) (layer "F.Cu") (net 9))
 (via (at 146.075 96.2) (size 0.8) (drill 0.4) (layers "F.Cu" "B.Cu") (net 9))
 (segment (start 148.995 99.12) (end 150.16 99.12) (width 0.25) (layer "B.Cu") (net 9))
 (segment (start 146.075 96.2) (end 148.995 99.12) (width 0.25) (layer "B.Cu") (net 9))
 (segment (start 136.2 90.4) (end 121 75.2) (width 0.25) (layer "F.Cu") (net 10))
 (segment (start 146.8 92.5) (end 144.7 90.4) (width 0.25) (layer "F.Cu") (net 10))
 (segment (start 146.8 98.1) (end 146.8 92.5) (width 0.25) (layer "F.Cu") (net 10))
 (segment (start 144.7 90.4) (end 136.2 90.4) (width 0.25) (layer "F.Cu") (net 10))
 (segment (start 146.8 98.1) (end 146.8 98.2) (width 0.25) (layer "F.Cu") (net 10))
 (segment (start 146.8 98.2) (end 146.774847 98.225153) (width 0.25) (layer "F.Cu") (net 10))
 (via (at 146.774847 98.225153) (size 0.8) (drill 0.4) (layers "F.Cu" "B.Cu") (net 10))
 (segment (start 146.774847 98.225153) (end 146.774847 98.274847) (width 0.25) (layer "B.Cu") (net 10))
 (segment (start 146.774847 98.274847) (end 150.16 101.66) (width 0.25) (layer "B.Cu") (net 10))
 (segment (start 161.4 105.66) (end 165.4 101.66) (width 0.25) (layer "F.Cu") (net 8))
 (segment (start 161.4 119.3) (end 161.4 105.66) (width 0.25) (layer "F.Cu") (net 8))
 (segment (start 111.4 104.4) (end 135.6 128.6) (width 0.25) (layer "F.Cu") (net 8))
 (segment (start 113 75.2) (end 111.4 76.8) (width 0.25) (layer "F.Cu") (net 8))
 (segment (start 152.1 128.6) (end 161.4 119.3) (width 0.25) (layer "F.Cu") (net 8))
 (segment (start 135.6 128.6) (end 152.1 128.6) (width 0.25) (layer "F.Cu") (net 8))
 (segment (start 111.4 76.8) (end 111.4 104.4) (width 0.25) (layer "F.Cu") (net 8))
 (segment (start 144.61 127.06) (end 150.16 127.06) (width 0.25) (layer "F.Cu") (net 19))
 (segment (start 142.7 125.15) (end 144.61 127.06) (width 0.25) (layer "F.Cu") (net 19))
 (segment (start 133.1 107.4) (end 137.275 107.4) (width 0.25) (layer "F.Cu") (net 57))
 (segment (start 133.1 104.9) (end 137.175 104.9) (width 0.25) (layer "F.Cu") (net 16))
 (segment (start 133.1 102.6) (end 137.275 102.6) (width 0.25) (layer "F.Cu") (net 17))
 (segment (start 143.4 100.5) (end 145.3 100.5) (width 0.25) (layer "F.Cu") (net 58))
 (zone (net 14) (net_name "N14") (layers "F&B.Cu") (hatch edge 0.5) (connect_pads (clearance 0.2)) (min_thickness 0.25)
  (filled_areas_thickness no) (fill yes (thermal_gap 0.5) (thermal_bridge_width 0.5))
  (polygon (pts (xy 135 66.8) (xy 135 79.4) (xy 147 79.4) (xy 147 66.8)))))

